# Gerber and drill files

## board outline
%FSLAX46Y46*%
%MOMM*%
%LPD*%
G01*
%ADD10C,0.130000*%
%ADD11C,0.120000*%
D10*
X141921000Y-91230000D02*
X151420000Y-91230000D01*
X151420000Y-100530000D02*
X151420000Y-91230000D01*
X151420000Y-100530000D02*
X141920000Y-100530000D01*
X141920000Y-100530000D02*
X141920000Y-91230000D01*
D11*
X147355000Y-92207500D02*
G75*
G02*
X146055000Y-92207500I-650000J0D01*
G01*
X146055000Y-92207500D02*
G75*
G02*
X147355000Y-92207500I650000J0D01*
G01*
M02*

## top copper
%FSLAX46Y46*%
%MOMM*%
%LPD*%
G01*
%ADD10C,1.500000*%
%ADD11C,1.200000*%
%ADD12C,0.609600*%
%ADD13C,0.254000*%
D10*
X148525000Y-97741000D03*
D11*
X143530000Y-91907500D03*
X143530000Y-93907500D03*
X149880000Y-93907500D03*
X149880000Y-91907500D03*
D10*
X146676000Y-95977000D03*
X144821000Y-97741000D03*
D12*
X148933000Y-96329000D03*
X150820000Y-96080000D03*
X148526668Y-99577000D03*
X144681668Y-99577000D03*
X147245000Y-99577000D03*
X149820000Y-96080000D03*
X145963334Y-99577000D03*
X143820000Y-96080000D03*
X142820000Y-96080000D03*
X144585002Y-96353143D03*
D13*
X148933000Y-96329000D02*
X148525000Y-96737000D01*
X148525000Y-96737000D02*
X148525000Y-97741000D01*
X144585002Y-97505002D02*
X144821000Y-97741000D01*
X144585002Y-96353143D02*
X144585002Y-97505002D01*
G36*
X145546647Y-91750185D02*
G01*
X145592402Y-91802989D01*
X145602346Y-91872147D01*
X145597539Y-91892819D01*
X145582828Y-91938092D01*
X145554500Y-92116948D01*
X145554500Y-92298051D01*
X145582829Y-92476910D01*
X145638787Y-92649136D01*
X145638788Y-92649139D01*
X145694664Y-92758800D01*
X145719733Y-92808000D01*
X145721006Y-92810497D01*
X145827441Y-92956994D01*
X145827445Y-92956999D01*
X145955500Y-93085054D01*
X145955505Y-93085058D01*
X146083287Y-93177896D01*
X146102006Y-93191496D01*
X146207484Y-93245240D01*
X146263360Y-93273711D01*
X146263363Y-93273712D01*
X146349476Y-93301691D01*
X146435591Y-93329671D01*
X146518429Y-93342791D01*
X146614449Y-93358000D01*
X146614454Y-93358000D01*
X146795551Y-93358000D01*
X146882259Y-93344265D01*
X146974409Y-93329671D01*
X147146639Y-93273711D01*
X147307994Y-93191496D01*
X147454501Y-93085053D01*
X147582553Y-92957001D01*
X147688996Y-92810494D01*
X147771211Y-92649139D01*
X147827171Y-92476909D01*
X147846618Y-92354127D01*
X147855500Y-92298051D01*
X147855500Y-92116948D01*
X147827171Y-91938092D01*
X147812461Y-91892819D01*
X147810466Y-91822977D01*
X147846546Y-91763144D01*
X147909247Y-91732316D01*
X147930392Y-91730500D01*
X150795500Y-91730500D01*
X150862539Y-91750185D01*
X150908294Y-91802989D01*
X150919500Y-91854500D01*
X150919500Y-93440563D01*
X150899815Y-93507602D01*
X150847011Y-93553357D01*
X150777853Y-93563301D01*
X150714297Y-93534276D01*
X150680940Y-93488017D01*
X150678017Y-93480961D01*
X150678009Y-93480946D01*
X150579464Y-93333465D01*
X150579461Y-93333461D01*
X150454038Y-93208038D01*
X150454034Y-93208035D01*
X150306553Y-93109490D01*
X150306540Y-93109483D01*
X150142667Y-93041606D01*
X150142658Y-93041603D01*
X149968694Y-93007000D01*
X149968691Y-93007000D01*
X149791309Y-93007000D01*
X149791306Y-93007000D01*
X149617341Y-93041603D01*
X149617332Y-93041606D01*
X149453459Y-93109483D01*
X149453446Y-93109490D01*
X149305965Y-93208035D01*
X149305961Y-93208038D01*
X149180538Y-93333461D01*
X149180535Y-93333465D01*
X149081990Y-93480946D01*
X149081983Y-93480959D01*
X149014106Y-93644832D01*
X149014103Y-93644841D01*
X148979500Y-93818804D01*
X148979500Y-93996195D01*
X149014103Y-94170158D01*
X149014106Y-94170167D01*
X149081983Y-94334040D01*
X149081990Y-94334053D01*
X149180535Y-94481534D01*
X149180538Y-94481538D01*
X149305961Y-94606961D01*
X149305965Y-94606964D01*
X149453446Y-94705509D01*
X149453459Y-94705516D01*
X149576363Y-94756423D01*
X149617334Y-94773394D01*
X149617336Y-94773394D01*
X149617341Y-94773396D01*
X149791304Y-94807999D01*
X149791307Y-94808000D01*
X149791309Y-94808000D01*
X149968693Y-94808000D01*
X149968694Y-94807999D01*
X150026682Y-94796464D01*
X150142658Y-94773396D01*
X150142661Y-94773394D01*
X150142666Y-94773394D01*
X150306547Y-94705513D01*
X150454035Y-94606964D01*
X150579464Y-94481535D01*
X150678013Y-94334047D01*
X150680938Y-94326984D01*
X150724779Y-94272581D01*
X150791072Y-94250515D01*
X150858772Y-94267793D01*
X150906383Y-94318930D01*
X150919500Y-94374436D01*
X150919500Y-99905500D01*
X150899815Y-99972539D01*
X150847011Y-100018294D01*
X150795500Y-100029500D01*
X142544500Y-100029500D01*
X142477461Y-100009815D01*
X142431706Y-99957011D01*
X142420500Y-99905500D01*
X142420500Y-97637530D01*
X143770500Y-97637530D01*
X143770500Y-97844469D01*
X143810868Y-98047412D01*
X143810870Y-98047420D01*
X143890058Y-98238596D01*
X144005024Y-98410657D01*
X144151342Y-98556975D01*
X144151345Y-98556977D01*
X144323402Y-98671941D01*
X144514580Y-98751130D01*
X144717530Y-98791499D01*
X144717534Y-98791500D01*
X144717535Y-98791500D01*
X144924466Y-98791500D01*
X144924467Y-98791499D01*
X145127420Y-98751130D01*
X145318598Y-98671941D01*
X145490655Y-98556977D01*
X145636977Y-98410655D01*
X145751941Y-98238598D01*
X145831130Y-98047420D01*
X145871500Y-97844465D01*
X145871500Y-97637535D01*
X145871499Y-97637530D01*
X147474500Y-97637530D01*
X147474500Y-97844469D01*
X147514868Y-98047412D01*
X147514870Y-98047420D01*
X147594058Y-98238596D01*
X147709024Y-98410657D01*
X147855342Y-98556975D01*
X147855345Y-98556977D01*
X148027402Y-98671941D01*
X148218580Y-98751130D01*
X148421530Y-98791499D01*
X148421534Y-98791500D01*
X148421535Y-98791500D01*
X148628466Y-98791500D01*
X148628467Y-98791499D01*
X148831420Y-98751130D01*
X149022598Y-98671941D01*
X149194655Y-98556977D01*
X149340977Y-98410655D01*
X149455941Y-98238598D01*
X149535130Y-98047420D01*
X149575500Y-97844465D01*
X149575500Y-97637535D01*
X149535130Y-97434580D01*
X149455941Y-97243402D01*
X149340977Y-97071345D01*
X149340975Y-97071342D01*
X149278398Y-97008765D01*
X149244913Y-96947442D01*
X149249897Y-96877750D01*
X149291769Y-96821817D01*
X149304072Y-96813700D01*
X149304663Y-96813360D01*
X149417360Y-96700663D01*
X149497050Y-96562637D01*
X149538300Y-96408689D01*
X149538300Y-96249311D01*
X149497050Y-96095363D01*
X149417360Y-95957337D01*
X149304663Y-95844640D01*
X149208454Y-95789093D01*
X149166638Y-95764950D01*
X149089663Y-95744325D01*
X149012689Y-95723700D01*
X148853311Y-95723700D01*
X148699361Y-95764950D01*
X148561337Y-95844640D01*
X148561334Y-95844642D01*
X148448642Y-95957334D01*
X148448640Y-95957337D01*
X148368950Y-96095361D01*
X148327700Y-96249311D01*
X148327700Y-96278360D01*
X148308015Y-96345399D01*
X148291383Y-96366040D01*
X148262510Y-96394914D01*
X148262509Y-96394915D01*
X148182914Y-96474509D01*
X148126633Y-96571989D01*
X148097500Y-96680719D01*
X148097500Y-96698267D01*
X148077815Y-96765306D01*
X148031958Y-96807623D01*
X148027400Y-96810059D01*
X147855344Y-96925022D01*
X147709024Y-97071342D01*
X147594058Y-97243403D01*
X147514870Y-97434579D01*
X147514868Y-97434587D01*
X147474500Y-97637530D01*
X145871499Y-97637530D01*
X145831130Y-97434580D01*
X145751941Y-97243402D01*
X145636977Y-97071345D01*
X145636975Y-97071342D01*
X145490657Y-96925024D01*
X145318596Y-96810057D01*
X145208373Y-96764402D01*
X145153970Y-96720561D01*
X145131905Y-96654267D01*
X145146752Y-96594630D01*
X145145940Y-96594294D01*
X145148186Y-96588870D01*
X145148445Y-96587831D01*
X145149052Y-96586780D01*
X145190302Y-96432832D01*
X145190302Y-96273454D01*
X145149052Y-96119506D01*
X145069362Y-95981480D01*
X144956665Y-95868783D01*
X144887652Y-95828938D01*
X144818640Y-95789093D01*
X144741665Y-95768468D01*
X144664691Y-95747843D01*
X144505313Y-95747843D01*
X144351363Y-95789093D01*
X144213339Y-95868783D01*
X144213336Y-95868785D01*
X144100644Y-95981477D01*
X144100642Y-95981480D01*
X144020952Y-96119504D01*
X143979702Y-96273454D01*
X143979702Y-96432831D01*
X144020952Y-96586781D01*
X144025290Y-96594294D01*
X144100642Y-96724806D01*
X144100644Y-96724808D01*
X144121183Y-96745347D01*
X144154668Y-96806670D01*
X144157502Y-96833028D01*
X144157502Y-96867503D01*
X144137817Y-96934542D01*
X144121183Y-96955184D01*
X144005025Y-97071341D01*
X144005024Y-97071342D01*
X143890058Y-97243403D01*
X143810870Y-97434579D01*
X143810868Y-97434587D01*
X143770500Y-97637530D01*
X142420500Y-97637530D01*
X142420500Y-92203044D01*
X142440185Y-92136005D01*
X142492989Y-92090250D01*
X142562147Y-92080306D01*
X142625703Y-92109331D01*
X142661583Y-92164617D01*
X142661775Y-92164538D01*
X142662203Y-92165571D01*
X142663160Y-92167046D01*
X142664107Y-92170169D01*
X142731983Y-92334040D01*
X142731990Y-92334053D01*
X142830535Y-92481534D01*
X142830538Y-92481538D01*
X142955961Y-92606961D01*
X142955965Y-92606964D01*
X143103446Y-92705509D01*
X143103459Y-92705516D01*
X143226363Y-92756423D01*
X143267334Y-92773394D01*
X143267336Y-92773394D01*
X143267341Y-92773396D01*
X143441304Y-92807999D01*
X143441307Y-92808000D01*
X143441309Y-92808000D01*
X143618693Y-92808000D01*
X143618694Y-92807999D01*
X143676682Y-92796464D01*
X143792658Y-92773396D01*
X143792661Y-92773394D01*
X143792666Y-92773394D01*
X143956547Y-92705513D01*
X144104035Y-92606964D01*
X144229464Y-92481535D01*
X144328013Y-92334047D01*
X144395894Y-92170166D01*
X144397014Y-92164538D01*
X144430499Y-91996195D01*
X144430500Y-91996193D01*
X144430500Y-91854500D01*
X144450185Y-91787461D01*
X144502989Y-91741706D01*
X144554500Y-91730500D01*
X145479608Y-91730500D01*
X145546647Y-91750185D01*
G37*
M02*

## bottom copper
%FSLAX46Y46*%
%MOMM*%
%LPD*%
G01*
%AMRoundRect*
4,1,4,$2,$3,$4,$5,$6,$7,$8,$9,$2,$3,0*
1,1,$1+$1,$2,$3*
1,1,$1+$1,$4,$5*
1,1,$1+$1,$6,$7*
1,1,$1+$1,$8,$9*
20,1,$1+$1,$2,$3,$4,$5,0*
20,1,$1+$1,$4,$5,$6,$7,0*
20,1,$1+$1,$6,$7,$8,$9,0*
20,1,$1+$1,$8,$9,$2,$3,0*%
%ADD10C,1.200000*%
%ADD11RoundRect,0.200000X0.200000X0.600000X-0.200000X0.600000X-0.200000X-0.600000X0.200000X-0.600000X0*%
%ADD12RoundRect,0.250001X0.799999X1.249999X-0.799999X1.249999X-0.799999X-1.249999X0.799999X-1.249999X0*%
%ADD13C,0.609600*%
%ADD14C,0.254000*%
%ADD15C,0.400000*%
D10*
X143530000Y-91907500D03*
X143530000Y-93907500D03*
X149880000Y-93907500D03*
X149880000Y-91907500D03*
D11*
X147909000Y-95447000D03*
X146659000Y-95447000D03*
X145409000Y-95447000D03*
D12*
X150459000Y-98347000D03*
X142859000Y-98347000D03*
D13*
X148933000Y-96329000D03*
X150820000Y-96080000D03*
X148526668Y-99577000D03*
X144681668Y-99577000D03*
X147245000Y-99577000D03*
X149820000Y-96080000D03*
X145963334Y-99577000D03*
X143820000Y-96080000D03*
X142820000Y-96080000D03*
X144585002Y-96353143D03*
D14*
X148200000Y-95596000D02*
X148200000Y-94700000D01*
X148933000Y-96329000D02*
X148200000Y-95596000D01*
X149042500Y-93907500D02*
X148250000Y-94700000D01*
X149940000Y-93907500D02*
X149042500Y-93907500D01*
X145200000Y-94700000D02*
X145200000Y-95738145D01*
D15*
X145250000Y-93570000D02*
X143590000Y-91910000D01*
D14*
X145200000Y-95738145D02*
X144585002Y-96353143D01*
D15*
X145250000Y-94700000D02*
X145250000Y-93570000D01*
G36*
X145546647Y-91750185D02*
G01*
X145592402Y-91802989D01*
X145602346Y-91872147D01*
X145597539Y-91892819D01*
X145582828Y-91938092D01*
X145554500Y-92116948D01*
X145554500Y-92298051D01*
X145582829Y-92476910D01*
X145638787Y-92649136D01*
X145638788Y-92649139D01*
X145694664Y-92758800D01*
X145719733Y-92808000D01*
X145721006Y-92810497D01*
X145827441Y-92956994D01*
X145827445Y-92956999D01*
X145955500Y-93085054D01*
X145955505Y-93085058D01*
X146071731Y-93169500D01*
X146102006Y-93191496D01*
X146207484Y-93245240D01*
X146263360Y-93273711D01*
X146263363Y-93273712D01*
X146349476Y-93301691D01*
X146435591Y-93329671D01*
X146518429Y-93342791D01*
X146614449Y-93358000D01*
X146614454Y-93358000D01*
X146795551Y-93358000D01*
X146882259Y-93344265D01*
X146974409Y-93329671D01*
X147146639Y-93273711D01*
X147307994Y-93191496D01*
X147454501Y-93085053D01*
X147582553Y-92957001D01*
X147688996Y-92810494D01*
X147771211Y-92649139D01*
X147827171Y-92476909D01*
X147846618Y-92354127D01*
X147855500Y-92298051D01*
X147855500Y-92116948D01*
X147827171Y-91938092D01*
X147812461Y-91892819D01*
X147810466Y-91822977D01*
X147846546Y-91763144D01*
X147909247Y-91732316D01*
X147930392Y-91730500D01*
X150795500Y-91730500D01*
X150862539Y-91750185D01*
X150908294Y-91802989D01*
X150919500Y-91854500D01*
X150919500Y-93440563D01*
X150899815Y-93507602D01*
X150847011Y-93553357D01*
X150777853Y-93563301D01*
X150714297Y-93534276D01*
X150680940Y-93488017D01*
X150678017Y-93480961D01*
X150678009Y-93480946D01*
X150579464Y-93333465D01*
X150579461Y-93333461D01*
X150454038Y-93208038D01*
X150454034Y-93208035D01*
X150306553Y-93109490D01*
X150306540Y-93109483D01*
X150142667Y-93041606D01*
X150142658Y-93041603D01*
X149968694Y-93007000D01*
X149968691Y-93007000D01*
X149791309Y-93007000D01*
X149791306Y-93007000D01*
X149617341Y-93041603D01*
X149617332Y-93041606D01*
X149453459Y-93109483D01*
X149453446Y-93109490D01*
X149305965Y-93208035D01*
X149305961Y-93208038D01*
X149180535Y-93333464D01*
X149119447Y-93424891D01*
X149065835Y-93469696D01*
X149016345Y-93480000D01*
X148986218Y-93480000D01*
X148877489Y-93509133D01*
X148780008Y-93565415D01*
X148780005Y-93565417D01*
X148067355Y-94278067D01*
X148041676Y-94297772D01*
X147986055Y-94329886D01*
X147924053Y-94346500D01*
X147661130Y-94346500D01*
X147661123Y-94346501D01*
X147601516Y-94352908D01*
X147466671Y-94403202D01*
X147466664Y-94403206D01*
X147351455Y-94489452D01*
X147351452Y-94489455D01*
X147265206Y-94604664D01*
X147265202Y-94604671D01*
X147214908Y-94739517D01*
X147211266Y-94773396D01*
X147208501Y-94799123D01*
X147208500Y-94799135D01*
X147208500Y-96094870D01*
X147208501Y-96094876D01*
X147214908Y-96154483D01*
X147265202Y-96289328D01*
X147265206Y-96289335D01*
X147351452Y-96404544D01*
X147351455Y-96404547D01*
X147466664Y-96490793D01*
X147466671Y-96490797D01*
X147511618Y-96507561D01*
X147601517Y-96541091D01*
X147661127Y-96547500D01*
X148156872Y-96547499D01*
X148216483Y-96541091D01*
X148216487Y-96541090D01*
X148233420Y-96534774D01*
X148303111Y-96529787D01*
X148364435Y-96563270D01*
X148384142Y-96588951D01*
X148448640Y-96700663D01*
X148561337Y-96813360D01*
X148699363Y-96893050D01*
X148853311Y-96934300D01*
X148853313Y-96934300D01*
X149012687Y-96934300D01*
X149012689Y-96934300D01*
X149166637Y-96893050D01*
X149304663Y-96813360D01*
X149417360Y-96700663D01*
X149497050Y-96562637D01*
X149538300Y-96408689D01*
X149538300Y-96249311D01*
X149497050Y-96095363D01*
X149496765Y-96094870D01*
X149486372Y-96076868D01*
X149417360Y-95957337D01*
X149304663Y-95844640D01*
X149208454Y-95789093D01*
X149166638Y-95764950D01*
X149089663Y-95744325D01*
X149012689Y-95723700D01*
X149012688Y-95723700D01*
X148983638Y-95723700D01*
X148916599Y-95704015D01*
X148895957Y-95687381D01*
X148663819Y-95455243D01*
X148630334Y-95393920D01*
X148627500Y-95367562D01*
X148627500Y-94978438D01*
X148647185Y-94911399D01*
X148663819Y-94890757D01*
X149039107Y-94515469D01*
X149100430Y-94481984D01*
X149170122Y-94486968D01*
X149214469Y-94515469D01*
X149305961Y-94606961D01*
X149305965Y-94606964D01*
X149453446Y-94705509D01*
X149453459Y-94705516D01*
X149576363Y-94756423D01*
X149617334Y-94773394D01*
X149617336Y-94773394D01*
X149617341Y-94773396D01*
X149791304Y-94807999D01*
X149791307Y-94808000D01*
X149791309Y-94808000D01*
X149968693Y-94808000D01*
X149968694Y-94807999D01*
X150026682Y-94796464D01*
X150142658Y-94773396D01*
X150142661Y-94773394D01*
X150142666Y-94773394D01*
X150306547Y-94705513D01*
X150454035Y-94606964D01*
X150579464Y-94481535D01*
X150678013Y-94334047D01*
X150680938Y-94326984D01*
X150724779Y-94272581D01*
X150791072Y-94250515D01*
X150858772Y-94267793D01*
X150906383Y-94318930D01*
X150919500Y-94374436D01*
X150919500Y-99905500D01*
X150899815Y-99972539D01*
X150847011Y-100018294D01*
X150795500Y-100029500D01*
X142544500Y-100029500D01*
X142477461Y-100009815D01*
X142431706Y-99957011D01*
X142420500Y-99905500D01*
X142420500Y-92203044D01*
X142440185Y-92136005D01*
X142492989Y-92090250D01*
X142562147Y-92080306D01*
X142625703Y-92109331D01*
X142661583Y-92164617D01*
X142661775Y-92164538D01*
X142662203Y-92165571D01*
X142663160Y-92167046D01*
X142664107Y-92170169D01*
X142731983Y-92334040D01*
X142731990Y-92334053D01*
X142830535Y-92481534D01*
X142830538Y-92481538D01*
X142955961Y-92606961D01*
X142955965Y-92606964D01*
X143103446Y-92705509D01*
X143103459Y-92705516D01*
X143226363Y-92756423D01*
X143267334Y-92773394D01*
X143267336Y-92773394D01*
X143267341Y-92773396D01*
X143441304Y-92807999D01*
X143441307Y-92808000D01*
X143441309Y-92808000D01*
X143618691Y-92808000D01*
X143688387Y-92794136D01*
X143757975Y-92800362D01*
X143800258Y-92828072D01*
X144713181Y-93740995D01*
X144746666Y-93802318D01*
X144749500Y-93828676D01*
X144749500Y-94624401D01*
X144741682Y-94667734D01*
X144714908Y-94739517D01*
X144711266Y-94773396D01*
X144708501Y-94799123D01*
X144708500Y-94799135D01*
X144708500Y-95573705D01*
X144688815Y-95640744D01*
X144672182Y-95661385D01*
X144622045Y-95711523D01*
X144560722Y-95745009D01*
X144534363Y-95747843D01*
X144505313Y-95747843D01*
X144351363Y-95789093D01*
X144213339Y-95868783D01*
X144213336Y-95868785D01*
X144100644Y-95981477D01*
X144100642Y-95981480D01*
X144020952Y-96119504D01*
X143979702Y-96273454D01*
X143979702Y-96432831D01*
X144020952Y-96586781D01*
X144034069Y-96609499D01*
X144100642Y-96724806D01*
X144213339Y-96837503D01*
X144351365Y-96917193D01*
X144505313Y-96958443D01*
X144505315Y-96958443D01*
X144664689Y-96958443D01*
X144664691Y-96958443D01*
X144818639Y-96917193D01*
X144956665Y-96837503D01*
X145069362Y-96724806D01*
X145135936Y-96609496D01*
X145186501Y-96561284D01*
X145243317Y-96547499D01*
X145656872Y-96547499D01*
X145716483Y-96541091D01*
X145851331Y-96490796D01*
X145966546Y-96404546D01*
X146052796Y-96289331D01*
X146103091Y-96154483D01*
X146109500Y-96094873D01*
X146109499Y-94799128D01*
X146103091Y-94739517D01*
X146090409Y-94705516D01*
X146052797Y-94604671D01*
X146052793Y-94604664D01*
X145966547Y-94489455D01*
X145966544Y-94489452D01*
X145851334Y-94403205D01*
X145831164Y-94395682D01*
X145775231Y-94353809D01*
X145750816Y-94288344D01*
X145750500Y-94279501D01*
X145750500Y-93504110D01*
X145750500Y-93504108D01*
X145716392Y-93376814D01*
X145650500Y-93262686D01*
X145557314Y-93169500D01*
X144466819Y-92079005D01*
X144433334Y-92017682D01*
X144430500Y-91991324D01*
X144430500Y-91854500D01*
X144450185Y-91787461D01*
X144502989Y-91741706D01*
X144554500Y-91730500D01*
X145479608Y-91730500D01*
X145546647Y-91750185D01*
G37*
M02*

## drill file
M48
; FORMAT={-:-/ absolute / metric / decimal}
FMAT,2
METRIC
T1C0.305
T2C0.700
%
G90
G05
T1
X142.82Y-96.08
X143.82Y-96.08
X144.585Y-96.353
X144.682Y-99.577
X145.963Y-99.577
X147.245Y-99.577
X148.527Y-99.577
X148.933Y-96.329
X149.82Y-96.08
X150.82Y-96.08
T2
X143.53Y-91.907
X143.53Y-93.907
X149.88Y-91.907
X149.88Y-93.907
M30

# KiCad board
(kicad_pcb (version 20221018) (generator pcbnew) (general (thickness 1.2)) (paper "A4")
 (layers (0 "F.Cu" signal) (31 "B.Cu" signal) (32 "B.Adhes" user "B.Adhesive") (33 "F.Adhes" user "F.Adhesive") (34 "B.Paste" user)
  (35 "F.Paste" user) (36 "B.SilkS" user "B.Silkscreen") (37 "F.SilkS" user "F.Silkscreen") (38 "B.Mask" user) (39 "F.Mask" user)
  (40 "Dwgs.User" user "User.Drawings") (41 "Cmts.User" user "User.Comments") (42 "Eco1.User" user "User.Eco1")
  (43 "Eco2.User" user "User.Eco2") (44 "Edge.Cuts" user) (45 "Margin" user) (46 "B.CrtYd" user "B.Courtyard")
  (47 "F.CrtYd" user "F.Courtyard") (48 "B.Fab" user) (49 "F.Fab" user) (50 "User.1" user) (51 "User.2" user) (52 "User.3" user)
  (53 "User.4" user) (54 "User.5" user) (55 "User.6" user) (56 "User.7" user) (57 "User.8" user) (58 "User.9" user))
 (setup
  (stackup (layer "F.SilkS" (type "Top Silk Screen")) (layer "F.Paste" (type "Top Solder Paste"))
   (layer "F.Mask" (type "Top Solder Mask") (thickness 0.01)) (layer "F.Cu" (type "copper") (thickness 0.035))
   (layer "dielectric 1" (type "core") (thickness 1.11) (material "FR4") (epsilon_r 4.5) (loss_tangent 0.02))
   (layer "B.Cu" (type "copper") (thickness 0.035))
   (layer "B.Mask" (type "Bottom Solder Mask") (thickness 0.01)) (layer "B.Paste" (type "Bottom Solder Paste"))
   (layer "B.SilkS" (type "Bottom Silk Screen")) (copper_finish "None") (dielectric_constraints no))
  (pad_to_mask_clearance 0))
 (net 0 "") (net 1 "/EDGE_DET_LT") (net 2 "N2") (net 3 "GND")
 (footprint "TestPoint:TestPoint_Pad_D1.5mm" (layer "F.Cu") (at 148.525 97.741)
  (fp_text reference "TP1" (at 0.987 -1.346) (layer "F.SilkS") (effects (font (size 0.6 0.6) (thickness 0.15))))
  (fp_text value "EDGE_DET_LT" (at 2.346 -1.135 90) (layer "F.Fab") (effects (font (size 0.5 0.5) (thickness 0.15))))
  (pad "1" smd circle (at 0 0) (size 1.5 1.5) (layers "F.Cu" "F.Mask") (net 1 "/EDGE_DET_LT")))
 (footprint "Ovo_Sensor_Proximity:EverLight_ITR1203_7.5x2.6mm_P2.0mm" (layer "F.Cu") (at 146.705 92.9075)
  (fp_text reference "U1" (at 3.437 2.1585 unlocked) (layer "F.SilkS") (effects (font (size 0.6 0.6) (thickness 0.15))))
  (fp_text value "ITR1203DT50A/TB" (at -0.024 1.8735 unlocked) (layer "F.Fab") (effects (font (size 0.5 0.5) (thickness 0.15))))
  (fp_circle (center 0 -0.7) (end 0.65 -0.7) (stroke (width 0.12) (type solid)) (fill none) (layer "Edge.Cuts"))
  (pad "1" thru_hole circle (at -3.175 -1) (size 1.2 1.2) (drill 0.7) (layers "*.Cu" "*.Mask") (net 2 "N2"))
  (pad "2" thru_hole circle (at -3.175 1) (size 1.2 1.2) (drill 0.7) (layers "*.Cu" "*.Mask") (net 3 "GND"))
  (pad "3" thru_hole circle (at 3.175 1) (size 1.2 1.2) (drill 0.7) (layers "*.Cu" "*.Mask") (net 1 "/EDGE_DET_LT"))
  (pad "4" thru_hole circle (at 3.175 -1) (size 1.2 1.2) (drill 0.7) (layers "*.Cu" "*.Mask") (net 3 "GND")))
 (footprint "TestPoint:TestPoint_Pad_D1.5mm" (layer "F.Cu") (at 146.676 95.977)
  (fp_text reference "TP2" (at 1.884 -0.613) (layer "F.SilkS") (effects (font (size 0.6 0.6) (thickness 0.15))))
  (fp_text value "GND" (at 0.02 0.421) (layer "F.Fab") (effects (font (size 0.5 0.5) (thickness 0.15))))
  (pad "1" smd circle (at 0 0) (size 1.5 1.5) (layers "F.Cu" "F.Mask") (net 3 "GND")))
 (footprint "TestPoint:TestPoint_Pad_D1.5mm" (layer "F.Cu") (at 144.821 97.741)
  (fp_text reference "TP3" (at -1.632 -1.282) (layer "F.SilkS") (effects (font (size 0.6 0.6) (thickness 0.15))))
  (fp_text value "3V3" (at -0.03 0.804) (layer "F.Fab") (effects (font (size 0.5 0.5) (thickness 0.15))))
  (pad "1" smd circle (at 0 0) (size 1.5 1.5) (layers "F.Cu" "F.Mask") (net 2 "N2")))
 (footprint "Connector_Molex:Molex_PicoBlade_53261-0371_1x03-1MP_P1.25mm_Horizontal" (layer "B.Cu") (at 146.659 97.847 180)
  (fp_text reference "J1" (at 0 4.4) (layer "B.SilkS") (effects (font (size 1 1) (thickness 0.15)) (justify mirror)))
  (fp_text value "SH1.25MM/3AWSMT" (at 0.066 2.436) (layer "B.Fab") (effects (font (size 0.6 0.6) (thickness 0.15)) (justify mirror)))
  (pad "1" smd roundrect (at -1.25 2.4 180) (size 0.8 1.6) (layers "B.Cu" "B.Paste" "B.Mask") (roundrect_rratio 0.25) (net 1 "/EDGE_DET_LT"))
  (pad "2" smd roundrect (at 0 2.4 180) (size 0.8 1.6) (layers "B.Cu" "B.Paste" "B.Mask") (roundrect_rratio 0.25) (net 3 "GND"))
  (pad "3" smd roundrect (at 1.25 2.4 180) (size 0.8 1.6) (layers "B.Cu" "B.Paste" "B.Mask") (roundrect_rratio 0.25) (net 2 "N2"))
  (pad "MP" smd roundrect (at -3.8 -0.5 180) (size 2.1 3) (layers "B.Cu" "B.Paste" "B.Mask") (roundrect_rratio 0.1190480952) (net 3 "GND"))
  (pad "MP" smd roundrect (at 3.8 -0.5 180) (size 2.1 3) (layers "B.Cu" "B.Paste" "B.Mask") (roundrect_rratio 0.1190480952) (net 3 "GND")))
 (gr_line (start 141.921 91.23) (end 151.42 91.23) (stroke (width 0.13) (type solid)) (layer "Edge.Cuts"))
 (gr_line (start 151.42 100.53) (end 151.42 91.23) (stroke (width 0.13) (type solid)) (layer "Edge.Cuts"))
 (gr_line (start 151.42 100.53) (end 141.92 100.53) (stroke (width 0.13) (type solid)) (layer "Edge.Cuts"))
 (gr_line (start 141.92 100.53) (end 141.92 91.23) (stroke (width 0.13) (type solid)) (layer "Edge.Cuts"))
 (segment (start 148.933 96.329) (end 148.525 96.737) (width 0.254) (layer "F.Cu") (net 1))
 (segment (start 148.525 96.737) (end 148.525 97.741) (width 0.254) (layer "F.Cu") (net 1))
 (via (at 148.933 96.329) (size 0.6096) (drill 0.3048) (layers "F.Cu" "B.Cu") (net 1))
 (segment (start 148.2 95.596) (end 148.2 94.7) (width 0.254) (layer "B.Cu") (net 1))
 (segment (start 148.933 96.329) (end 148.2 95.596) (width 0.254) (layer "B.Cu") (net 1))
 (segment (start 149.0425 93.9075) (end 148.25 94.7) (width 0.254) (layer "B.Cu") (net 1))
 (segment (start 149.94 93.9075) (end 149.0425 93.9075) (width 0.254) (layer "B.Cu") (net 1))
 (via (at 150.82 96.08) (size 0.6096) (drill 0.3048) (layers "F.Cu" "B.Cu") (free) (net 3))
 (via (at 148.526668 99.577) (size 0.6096) (drill 0.3048) (layers "F.Cu" "B.Cu") (free) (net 3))
 (via (at 144.681668 99.577) (size 0.6096) (drill 0.3048) (layers "F.Cu" "B.Cu") (free) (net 3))
 (via (at 147.245 99.577) (size 0.6096) (drill 0.3048) (layers "F.Cu" "B.Cu") (free) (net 3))
 (via (at 149.82 96.08) (size 0.6096) (drill 0.3048) (layers "F.Cu" "B.Cu") (free) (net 3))
 (via (at 145.963334 99.577) (size 0.6096) (drill 0.3048) (layers "F.Cu" "B.Cu") (free) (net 3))
 (via (at 143.82 96.08) (size 0.6096) (drill 0.3048) (layers "F.Cu" "B.Cu") (free) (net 3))
 (via (at 142.82 96.08) (size 0.6096) (drill 0.3048) (layers "F.Cu" "B.Cu") (free) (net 3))
 (segment (start 144.585002 97.505002) (end 144.821 97.741) (width 0.254) (layer "F.Cu") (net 2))
 (segment (start 144.585002 96.353143) (end 144.585002 97.505002) (width 0.254) (layer "F.Cu") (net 2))
 (via (at 144.585002 96.353143) (size 0.6096) (drill 0.3048) (layers "F.Cu" "B.Cu") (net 2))
 (segment (start 145.2 94.7) (end 145.2 95.738145) (width 0.254) (layer "B.Cu") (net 2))
 (segment (start 145.25 93.57) (end 143.59 91.91) (width 0.4) (layer "B.Cu") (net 2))
 (segment (start 145.2 95.738145) (end 144.585002 96.353143) (width 0.254) (layer "B.Cu") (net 2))
 (segment (start 145.25 94.7) (end 145.25 93.57) (width 0.4) (layer "B.Cu") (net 2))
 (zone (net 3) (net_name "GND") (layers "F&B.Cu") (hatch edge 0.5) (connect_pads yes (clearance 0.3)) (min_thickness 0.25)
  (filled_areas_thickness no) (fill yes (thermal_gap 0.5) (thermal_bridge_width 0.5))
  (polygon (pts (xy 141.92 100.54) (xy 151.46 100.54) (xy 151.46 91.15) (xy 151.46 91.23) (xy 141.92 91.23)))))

